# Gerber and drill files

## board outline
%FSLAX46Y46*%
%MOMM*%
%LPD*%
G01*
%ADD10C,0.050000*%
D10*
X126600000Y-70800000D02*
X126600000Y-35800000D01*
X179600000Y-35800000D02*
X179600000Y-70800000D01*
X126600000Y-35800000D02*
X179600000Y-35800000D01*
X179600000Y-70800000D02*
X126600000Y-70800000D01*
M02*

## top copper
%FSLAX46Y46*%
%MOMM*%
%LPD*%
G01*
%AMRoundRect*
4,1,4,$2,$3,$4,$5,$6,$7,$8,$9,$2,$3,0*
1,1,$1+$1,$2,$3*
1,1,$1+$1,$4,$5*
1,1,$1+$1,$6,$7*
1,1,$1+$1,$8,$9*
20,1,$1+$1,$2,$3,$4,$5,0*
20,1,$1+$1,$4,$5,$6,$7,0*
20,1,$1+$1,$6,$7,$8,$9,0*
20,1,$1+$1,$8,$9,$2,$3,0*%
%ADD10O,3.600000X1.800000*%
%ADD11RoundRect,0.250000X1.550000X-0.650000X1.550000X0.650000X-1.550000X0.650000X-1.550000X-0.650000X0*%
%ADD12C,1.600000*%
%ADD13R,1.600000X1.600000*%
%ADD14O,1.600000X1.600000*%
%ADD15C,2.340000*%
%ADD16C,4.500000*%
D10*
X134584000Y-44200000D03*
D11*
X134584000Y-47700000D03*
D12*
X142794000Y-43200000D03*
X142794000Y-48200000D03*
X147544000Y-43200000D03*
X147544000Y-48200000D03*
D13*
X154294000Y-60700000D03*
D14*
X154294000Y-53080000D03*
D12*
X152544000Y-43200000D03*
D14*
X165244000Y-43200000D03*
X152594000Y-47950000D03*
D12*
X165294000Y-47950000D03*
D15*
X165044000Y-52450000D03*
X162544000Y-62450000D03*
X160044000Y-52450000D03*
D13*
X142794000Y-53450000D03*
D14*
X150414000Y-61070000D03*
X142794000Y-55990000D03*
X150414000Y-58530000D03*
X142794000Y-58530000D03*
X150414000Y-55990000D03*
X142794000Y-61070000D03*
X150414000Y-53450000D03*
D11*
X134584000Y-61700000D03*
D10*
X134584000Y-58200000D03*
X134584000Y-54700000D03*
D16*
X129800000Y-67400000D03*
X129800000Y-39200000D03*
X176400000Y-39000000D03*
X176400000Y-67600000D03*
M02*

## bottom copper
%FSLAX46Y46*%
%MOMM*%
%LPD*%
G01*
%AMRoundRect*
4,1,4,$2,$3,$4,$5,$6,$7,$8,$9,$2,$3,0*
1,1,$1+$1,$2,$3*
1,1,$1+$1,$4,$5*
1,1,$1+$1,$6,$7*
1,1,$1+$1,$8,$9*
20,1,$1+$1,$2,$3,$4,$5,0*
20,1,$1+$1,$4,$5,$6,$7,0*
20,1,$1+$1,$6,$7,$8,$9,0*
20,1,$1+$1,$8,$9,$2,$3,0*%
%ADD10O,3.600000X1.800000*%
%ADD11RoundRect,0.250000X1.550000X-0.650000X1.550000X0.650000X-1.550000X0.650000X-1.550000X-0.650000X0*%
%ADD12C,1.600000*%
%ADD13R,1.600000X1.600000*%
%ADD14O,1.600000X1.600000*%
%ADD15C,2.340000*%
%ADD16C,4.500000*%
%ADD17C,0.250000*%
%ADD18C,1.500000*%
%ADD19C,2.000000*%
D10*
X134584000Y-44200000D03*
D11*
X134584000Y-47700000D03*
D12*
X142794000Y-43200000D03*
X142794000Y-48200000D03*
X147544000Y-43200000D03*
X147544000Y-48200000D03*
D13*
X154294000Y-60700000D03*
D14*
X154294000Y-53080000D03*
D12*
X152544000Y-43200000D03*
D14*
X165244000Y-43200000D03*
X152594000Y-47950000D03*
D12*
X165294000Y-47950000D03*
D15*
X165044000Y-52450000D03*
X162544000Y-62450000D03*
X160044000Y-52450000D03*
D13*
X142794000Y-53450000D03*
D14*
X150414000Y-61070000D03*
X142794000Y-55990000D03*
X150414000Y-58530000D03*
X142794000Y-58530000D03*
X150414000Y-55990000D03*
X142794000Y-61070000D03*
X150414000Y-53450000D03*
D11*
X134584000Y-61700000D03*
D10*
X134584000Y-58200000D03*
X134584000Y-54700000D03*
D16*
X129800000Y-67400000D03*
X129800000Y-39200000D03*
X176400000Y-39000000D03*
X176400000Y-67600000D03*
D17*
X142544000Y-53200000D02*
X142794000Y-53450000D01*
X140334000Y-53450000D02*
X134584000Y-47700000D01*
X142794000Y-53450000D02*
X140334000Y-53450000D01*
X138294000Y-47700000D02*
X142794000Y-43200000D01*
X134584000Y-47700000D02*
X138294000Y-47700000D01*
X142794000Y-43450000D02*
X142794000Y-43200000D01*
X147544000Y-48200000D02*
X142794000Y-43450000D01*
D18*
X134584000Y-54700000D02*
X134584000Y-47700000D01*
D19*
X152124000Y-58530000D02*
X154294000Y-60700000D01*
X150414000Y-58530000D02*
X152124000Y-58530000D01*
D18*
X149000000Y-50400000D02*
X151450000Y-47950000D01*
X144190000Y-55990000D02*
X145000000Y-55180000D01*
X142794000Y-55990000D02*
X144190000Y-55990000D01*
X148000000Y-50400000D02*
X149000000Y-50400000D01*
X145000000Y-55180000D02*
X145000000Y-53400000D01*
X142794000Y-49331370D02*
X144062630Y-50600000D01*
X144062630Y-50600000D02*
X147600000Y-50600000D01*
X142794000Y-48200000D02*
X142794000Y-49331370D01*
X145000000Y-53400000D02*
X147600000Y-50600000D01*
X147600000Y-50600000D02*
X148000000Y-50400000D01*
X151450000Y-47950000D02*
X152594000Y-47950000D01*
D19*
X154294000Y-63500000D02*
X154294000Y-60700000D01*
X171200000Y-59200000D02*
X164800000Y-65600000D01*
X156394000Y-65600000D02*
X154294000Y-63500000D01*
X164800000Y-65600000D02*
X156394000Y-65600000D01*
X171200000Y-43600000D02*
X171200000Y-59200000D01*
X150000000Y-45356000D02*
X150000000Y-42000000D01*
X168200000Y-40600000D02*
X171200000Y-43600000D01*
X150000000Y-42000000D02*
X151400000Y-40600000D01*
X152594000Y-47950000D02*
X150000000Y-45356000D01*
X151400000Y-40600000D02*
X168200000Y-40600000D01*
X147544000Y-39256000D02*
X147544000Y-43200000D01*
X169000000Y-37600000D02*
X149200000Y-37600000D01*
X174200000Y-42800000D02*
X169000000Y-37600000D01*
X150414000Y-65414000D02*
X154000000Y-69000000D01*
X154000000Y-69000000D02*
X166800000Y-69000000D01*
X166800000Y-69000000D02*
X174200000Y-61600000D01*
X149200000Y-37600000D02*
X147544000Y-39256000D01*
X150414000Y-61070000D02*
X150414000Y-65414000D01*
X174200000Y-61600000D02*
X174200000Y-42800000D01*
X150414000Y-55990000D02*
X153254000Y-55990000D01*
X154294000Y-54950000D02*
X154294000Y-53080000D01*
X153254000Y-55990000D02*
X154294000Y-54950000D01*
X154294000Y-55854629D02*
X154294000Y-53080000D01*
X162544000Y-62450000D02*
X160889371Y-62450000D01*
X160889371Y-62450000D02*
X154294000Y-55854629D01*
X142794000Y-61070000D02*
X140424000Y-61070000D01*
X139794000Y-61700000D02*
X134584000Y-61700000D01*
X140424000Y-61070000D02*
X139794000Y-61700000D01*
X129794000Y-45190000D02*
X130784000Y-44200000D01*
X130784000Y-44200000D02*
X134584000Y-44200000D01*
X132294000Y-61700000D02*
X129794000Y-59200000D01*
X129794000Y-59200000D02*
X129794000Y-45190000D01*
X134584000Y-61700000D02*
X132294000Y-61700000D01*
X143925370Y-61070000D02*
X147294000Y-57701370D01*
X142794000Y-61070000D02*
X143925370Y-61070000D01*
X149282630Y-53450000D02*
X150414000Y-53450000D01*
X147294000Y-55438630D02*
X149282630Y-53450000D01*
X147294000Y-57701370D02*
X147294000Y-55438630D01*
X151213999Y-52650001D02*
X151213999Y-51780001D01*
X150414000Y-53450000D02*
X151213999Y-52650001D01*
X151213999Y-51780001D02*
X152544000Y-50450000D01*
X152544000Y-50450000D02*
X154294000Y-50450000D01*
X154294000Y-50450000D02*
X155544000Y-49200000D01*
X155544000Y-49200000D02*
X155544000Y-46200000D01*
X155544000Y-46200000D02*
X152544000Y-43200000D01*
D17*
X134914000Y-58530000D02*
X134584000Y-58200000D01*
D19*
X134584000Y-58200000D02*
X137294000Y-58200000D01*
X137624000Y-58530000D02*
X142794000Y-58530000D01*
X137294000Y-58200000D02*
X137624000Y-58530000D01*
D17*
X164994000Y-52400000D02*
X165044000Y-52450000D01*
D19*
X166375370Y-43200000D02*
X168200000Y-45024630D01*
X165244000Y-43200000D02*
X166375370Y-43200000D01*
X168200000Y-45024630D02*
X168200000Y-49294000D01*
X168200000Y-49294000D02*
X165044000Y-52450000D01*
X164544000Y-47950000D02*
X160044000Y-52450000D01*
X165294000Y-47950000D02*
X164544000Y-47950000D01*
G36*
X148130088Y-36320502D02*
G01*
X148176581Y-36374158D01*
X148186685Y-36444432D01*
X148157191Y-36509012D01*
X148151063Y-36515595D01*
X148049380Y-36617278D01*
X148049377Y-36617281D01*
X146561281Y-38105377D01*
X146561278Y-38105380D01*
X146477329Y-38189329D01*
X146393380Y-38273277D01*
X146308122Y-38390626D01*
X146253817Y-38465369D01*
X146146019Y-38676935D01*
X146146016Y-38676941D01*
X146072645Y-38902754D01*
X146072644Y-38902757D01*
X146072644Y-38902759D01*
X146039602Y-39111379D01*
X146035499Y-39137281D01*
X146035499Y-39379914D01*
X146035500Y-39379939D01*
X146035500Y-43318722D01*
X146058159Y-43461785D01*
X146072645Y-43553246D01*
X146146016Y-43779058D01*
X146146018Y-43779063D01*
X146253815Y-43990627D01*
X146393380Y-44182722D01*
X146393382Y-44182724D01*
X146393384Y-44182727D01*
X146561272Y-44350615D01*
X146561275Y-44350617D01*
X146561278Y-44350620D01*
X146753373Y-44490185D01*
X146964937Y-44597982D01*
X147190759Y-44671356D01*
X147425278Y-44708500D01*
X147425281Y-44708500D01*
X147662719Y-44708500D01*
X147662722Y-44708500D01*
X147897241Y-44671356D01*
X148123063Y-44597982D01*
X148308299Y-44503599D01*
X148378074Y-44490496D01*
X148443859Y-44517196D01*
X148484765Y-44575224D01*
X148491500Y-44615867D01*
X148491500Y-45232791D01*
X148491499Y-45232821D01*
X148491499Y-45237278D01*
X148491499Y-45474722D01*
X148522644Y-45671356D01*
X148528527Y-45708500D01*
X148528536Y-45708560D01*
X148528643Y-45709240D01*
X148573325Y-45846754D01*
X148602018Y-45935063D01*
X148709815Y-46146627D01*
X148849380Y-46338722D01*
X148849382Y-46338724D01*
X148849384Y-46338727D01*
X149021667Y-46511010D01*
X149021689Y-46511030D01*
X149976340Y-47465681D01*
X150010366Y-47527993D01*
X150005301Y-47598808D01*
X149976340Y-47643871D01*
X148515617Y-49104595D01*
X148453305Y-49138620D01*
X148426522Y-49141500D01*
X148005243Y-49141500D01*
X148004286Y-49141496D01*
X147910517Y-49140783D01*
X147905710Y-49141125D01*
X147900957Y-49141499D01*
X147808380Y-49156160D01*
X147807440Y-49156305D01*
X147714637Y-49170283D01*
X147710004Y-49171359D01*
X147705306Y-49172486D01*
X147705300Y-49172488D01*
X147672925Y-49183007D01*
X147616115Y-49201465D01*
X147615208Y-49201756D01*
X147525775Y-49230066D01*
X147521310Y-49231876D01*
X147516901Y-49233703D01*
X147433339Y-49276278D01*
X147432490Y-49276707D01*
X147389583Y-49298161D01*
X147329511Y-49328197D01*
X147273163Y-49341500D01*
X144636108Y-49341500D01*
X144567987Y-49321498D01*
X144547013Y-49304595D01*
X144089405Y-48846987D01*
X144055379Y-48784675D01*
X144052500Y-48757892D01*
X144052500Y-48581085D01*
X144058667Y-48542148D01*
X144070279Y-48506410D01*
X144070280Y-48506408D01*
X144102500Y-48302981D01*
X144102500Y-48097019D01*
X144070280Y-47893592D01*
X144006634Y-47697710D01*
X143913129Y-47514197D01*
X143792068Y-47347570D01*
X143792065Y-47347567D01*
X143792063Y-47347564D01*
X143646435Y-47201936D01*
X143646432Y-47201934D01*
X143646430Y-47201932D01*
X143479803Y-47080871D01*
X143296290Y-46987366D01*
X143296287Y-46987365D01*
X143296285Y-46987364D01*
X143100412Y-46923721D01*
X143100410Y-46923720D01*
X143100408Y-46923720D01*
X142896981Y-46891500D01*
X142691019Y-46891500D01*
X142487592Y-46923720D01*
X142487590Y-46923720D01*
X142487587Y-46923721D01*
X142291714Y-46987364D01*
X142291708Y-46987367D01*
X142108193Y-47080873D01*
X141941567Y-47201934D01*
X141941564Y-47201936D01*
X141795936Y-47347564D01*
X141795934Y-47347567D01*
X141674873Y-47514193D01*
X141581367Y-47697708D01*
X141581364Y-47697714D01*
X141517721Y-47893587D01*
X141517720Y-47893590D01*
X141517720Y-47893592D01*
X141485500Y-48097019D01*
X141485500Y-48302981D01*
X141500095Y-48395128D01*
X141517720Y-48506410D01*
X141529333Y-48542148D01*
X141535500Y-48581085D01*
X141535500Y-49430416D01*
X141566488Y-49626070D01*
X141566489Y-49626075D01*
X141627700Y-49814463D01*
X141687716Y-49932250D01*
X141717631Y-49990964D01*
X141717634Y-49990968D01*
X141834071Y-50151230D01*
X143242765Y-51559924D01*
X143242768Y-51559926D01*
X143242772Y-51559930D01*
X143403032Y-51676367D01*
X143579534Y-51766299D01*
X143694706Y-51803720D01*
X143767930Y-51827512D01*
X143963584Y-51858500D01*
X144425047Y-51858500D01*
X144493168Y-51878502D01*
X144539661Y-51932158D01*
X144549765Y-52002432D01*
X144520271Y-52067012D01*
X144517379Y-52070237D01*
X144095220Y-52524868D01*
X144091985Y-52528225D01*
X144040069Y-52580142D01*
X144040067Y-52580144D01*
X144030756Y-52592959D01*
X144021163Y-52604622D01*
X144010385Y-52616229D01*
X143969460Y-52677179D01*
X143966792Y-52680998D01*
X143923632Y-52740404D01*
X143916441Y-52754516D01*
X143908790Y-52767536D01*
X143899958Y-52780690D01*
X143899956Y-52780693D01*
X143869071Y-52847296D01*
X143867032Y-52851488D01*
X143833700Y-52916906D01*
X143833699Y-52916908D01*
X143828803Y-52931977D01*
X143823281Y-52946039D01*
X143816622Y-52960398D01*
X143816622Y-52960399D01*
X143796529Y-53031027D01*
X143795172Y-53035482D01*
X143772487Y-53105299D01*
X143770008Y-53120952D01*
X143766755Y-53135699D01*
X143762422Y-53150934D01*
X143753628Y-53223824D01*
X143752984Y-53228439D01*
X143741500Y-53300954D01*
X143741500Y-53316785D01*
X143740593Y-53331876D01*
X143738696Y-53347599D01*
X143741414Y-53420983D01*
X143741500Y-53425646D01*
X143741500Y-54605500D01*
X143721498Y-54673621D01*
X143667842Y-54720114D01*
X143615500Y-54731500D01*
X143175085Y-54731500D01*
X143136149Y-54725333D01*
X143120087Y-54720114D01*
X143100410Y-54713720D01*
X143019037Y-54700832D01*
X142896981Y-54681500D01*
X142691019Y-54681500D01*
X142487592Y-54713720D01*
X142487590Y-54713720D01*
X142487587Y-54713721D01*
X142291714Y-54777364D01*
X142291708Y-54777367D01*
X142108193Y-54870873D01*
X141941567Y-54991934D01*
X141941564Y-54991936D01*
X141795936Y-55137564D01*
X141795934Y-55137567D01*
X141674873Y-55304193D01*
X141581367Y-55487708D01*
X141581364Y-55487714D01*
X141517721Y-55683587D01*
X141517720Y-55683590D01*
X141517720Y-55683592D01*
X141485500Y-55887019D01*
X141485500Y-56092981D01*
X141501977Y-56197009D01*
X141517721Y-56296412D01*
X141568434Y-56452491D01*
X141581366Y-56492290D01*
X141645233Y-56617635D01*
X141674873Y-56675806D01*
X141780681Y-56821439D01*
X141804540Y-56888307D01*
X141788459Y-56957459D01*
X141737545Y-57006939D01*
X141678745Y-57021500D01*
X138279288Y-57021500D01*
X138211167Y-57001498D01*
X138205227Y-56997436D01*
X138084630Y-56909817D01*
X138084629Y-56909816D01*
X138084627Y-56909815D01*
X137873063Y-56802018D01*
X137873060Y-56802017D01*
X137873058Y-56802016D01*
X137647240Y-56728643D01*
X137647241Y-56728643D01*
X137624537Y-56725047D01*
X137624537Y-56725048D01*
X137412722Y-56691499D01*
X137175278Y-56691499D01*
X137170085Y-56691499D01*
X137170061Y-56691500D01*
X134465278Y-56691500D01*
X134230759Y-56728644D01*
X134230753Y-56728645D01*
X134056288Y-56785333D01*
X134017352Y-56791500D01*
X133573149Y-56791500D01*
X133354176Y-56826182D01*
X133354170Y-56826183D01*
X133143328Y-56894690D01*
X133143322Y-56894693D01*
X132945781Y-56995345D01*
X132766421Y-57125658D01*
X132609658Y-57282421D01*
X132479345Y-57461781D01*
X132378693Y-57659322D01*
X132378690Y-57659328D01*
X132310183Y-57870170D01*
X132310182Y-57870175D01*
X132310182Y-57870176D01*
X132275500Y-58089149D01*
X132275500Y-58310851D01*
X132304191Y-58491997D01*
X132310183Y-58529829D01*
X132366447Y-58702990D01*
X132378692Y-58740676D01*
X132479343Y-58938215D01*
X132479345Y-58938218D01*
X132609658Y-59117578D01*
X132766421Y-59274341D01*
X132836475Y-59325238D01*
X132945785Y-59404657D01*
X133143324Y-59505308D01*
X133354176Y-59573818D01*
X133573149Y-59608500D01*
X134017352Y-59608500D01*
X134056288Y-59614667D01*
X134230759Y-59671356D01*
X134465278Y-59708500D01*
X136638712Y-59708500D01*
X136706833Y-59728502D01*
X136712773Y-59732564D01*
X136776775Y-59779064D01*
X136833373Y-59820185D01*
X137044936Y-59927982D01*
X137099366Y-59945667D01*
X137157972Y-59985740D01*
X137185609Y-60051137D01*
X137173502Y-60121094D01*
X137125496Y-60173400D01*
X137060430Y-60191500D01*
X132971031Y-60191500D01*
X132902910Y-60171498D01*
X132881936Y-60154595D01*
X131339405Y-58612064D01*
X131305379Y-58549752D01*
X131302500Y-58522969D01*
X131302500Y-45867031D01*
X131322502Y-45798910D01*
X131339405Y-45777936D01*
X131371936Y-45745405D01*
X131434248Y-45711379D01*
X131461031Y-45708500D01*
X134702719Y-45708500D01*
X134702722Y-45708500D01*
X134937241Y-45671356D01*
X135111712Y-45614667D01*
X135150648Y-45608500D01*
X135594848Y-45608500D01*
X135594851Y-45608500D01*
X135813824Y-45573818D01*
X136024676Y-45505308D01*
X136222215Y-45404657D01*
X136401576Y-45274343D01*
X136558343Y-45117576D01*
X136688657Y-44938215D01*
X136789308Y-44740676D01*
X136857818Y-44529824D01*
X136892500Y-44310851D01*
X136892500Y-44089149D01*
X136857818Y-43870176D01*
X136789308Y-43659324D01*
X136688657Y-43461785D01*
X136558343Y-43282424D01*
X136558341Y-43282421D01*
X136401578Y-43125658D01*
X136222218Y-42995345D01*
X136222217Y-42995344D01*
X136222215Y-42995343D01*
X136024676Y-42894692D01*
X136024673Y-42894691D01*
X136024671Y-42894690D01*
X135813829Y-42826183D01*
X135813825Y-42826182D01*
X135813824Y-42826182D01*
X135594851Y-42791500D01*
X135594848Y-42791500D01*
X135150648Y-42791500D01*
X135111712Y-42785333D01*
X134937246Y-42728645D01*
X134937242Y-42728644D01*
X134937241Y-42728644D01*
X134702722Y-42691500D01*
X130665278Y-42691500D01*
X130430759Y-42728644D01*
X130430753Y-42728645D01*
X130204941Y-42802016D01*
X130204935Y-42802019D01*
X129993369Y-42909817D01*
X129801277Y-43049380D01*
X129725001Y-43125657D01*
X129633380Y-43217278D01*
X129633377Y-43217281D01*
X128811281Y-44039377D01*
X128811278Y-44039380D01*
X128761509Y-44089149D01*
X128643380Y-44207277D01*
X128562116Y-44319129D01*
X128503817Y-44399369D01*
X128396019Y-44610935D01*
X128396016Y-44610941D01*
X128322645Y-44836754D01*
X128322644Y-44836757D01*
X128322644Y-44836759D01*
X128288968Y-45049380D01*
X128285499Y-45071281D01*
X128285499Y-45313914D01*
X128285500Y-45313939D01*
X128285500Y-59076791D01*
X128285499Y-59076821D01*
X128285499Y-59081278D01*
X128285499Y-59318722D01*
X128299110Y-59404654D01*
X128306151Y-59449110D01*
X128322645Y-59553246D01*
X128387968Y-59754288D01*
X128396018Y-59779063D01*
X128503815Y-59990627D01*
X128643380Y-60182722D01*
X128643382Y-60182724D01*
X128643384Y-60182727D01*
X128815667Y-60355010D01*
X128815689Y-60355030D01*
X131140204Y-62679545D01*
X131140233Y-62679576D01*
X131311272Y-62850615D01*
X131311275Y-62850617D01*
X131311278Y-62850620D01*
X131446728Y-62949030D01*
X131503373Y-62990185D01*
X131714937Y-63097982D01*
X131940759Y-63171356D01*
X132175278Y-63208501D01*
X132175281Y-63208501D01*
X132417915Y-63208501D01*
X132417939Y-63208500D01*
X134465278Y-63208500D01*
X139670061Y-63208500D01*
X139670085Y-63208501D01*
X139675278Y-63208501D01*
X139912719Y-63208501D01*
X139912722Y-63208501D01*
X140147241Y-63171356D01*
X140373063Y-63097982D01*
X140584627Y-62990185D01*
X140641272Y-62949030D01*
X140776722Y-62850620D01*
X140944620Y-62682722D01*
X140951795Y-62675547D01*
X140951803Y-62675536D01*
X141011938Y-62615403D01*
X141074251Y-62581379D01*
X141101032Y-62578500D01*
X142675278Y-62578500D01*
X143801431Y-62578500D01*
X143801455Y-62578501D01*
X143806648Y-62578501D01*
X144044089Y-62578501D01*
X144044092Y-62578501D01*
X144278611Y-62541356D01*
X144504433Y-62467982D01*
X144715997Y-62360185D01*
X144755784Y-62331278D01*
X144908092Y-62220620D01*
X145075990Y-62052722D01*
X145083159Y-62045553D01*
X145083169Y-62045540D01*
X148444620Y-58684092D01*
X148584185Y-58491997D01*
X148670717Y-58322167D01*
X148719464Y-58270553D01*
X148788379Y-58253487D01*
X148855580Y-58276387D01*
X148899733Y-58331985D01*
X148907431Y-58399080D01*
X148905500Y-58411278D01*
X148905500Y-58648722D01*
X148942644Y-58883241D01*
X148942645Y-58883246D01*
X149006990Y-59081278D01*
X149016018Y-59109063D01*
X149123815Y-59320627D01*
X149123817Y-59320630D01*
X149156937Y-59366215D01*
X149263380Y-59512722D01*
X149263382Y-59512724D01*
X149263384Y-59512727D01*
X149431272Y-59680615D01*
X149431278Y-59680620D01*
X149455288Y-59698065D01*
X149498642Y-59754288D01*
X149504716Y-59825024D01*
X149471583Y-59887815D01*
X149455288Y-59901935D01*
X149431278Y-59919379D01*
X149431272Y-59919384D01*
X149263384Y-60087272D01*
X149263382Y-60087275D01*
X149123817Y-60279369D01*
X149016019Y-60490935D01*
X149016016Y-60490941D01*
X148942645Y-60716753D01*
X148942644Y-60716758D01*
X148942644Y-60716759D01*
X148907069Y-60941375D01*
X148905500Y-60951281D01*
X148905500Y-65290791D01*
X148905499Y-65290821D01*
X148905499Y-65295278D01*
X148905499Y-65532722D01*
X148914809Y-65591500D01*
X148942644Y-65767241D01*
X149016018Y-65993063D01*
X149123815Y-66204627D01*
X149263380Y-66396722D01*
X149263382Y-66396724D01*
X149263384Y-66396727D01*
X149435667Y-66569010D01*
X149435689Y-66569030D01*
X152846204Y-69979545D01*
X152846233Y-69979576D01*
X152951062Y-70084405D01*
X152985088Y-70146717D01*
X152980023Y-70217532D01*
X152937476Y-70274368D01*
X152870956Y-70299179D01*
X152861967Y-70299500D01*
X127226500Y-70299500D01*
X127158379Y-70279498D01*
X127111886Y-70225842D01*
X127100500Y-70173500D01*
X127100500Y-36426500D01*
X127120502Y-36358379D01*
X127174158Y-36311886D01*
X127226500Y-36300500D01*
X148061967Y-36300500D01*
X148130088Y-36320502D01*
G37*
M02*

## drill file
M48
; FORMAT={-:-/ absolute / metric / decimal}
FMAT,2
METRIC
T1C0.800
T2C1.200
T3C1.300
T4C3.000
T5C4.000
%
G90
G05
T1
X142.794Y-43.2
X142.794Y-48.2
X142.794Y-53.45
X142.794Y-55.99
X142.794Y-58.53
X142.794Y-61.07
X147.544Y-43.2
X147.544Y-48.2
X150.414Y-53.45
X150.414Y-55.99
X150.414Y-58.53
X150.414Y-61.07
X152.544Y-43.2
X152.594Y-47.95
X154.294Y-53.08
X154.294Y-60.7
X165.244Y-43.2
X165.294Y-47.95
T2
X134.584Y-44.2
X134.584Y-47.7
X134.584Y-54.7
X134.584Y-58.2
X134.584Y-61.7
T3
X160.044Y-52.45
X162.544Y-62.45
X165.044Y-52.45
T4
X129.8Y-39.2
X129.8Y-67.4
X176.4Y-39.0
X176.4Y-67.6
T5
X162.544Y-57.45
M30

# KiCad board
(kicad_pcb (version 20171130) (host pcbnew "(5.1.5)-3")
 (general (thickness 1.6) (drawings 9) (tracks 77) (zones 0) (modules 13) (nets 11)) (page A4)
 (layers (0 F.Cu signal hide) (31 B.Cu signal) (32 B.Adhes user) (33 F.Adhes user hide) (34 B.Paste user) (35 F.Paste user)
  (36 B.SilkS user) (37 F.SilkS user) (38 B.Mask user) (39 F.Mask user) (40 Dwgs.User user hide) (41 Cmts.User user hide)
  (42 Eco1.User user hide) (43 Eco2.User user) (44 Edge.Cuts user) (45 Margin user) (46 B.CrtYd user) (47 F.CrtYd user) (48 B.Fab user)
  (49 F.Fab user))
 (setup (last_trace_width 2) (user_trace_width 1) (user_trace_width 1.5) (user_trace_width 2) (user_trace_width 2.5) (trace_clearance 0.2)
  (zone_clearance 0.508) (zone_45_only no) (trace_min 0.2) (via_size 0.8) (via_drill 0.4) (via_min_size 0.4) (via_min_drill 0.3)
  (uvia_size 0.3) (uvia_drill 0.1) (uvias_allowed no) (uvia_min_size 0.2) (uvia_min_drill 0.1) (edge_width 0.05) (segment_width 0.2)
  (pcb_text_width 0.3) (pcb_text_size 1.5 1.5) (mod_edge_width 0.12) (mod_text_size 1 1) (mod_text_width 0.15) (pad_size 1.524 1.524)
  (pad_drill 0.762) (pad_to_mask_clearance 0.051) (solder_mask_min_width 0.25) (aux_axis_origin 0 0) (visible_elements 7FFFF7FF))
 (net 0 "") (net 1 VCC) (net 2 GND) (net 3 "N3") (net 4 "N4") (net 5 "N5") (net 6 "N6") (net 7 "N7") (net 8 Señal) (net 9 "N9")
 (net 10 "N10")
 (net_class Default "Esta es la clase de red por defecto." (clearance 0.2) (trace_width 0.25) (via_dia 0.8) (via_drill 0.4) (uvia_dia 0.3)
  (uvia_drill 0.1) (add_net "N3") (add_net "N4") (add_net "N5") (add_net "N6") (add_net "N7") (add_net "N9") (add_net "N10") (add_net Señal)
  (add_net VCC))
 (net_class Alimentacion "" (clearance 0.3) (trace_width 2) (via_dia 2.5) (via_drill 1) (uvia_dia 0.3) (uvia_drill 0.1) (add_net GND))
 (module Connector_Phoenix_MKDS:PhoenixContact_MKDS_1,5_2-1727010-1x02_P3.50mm (layer F.Cu) (at 132.044 47.7 90)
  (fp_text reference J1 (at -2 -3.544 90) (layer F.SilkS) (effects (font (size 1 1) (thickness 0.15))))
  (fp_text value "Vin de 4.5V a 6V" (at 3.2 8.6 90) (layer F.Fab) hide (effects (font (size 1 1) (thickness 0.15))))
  (pad 2 thru_hole oval (at 3.5 2.54 90) (size 1.8 3.6) (drill 1.2) (layers *.Cu *.Mask) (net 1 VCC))
  (pad 1 thru_hole roundrect (at 0 2.54 90) (size 1.8 3.6) (drill 1.2) (layers *.Cu *.Mask) (roundrect_rratio 0.138889) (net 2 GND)))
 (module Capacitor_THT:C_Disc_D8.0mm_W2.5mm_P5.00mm (layer F.Cu) (at 142.794 48.2 90)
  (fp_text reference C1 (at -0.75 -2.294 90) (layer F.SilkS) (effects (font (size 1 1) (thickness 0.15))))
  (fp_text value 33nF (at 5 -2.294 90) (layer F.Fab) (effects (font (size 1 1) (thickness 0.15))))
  (pad 2 thru_hole circle (at 5 0 90) (size 1.6 1.6) (drill 0.8) (layers *.Cu *.Mask) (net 2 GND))
  (pad 1 thru_hole circle (at 0 0 90) (size 1.6 1.6) (drill 0.8) (layers *.Cu *.Mask) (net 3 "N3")))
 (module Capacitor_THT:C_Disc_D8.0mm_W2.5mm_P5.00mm (layer F.Cu) (at 147.544 43.2 270)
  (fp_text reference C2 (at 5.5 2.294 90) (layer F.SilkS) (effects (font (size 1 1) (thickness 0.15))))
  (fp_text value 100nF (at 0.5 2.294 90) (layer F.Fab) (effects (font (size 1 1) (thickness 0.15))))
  (pad 1 thru_hole circle (at 0 0 270) (size 1.6 1.6) (drill 0.8) (layers *.Cu *.Mask) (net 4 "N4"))
  (pad 2 thru_hole circle (at 5 0 270) (size 1.6 1.6) (drill 0.8) (layers *.Cu *.Mask) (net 2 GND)))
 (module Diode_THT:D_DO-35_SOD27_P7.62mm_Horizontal (layer F.Cu) (at 154.294 60.7 90)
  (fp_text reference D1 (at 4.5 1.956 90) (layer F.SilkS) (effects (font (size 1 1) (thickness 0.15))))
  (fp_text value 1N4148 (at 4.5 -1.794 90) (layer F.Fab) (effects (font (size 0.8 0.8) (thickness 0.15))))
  (pad 1 thru_hole rect (at 0 0 90) (size 1.6 1.6) (drill 0.8) (layers *.Cu *.Mask) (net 3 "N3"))
  (pad 2 thru_hole oval (at 7.62 0 90) (size 1.6 1.6) (drill 0.8) (layers *.Cu *.Mask) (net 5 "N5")))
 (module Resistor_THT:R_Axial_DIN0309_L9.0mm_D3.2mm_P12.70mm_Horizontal (layer F.Cu) (at 152.544 43.2)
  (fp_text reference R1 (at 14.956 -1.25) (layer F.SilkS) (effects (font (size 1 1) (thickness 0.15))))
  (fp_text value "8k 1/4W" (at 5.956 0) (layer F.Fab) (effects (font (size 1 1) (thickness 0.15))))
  (pad 1 thru_hole circle (at 0 0) (size 1.6 1.6) (drill 0.8) (layers *.Cu *.Mask) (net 1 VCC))
  (pad 2 thru_hole oval (at 12.7 0) (size 1.6 1.6) (drill 0.8) (layers *.Cu *.Mask) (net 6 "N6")))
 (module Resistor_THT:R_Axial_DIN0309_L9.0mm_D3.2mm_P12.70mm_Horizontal (layer F.Cu) (at 165.294 47.95 180)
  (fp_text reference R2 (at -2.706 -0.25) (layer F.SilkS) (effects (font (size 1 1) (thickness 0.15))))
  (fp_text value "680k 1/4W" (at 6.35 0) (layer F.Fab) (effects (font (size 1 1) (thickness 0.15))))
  (pad 2 thru_hole oval (at 12.7 0 180) (size 1.6 1.6) (drill 0.8) (layers *.Cu *.Mask) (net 3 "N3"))
  (pad 1 thru_hole circle (at 0 0 180) (size 1.6 1.6) (drill 0.8) (layers *.Cu *.Mask) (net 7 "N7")))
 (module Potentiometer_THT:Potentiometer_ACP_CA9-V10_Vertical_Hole (layer F.Cu) (at 160.044 52.45 270)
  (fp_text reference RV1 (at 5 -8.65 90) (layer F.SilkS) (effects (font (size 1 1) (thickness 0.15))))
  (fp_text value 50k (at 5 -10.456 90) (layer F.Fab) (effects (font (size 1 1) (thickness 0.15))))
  (pad 3 thru_hole circle (at 0 -5 270) (size 2.34 2.34) (drill 1.3) (layers *.Cu *.Mask) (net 6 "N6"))
  (pad 2 thru_hole circle (at 10 -2.5 270) (size 2.34 2.34) (drill 1.3) (layers *.Cu *.Mask) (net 5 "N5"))
  (pad 1 thru_hole circle (at 0 0 270) (size 2.34 2.34) (drill 1.3) (layers *.Cu *.Mask) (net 7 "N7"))
  (pad "" np_thru_hole circle (at 5 -2.5 270) (size 4 4) (drill 4) (layers *.Cu *.Mask)))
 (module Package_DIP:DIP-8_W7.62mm (layer F.Cu) (at 142.794 53.45)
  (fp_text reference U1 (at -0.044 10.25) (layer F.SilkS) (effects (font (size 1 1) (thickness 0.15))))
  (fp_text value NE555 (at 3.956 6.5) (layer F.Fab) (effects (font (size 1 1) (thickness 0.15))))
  (pad 1 thru_hole rect (at 0 0) (size 1.6 1.6) (drill 0.8) (layers *.Cu *.Mask) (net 2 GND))
  (pad 5 thru_hole oval (at 7.62 7.62) (size 1.6 1.6) (drill 0.8) (layers *.Cu *.Mask) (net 4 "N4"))
  (pad 2 thru_hole oval (at 0 2.54) (size 1.6 1.6) (drill 0.8) (layers *.Cu *.Mask) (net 3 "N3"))
  (pad 6 thru_hole oval (at 7.62 5.08) (size 1.6 1.6) (drill 0.8) (layers *.Cu *.Mask) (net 3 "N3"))
  (pad 3 thru_hole oval (at 0 5.08) (size 1.6 1.6) (drill 0.8) (layers *.Cu *.Mask) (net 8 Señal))
  (pad 7 thru_hole oval (at 7.62 2.54) (size 1.6 1.6) (drill 0.8) (layers *.Cu *.Mask) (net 5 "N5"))
  (pad 4 thru_hole oval (at 0 7.62) (size 1.6 1.6) (drill 0.8) (layers *.Cu *.Mask) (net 1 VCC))
  (pad 8 thru_hole oval (at 7.62 0) (size 1.6 1.6) (drill 0.8) (layers *.Cu *.Mask) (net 1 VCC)))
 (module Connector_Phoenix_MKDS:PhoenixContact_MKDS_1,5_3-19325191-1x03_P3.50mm (layer F.Cu) (at 132.044 61.7 90)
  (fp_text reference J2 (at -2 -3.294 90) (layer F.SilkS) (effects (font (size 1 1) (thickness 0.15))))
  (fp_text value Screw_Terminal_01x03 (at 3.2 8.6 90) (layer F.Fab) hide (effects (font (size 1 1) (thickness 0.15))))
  (pad 1 thru_hole roundrect (at 0 2.54 90) (size 1.8 3.6) (drill 1.2) (layers *.Cu *.Mask) (roundrect_rratio 0.138889) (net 1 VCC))
  (pad 2 thru_hole oval (at 3.5 2.54 90) (size 1.8 3.6) (drill 1.2) (layers *.Cu *.Mask) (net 8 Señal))
  (pad 3 thru_hole oval (at 7 2.54 90) (size 1.8 3.6) (drill 1.2) (layers *.Cu *.Mask) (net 2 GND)))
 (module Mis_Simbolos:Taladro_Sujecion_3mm (layer F.Cu) (at 129.8 67.4)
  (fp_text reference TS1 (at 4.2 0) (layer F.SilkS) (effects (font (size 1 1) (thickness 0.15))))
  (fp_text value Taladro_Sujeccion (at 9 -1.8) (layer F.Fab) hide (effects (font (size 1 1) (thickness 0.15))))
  (pad 1 thru_hole circle (at 0 0) (size 4.5 4.5) (drill 3) (layers *.Cu *.Mask) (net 2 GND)))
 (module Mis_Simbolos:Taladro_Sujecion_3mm (layer F.Cu) (at 129.8 39.2)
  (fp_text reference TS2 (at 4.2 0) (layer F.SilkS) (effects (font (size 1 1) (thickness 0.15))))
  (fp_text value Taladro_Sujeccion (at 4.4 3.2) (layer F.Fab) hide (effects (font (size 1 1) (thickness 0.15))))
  (pad 1 thru_hole circle (at 0 0) (size 4.5 4.5) (drill 3) (layers *.Cu *.Mask) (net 2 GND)))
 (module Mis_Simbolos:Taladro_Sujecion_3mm (layer F.Cu) (at 176.4 39)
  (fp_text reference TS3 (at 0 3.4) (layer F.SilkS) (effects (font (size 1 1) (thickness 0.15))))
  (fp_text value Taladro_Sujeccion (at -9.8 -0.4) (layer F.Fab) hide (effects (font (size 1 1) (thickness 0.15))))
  (pad 1 thru_hole circle (at 0 0) (size 4.5 4.5) (drill 3) (layers *.Cu *.Mask) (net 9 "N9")))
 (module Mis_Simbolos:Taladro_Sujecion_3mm (layer F.Cu) (at 176.4 67.6)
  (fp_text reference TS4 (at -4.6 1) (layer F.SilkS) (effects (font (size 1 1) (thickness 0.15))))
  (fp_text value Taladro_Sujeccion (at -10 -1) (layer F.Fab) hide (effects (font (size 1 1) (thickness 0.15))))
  (pad 1 thru_hole circle (at 0 0) (size 4.5 4.5) (drill 3) (layers *.Cu *.Mask) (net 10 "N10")))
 (gr_line (start 126.6 70.8) (end 126.6 35.8) (layer Edge.Cuts) (width 0.05))
 (gr_line (start 179.6 35.8) (end 179.6 70.8) (layer Edge.Cuts) (width 0.05))
 (gr_line (start 126.6 35.8) (end 179.6 35.8) (layer Edge.Cuts) (width 0.05))
 (gr_line (start 179.6 70.8) (end 126.6 70.8) (layer Edge.Cuts) (width 0.05))
 (segment (start 142.544 53.2) (end 142.794 53.45) (width 0.25) (layer B.Cu) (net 2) (status 30))
 (segment (start 140.334 53.45) (end 134.584 47.7) (width 0.25) (layer B.Cu) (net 2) (status 20))
 (segment (start 142.794 53.45) (end 140.334 53.45) (width 0.25) (layer B.Cu) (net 2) (status 10))
 (segment (start 138.294 47.7) (end 142.794 43.2) (width 0.25) (layer B.Cu) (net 2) (status 20))
 (segment (start 134.584 47.7) (end 138.294 47.7) (width 0.25) (layer B.Cu) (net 2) (status 10))
 (segment (start 142.794 43.45) (end 142.794 43.2) (width 0.25) (layer B.Cu) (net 2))
 (segment (start 147.544 48.2) (end 142.794 43.45) (width 0.25) (layer B.Cu) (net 2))
 (segment (start 134.584 54.7) (end 134.584 47.7) (width 1.5) (layer B.Cu) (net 2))
 (segment (start 152.124 58.53) (end 154.294 60.7) (width 2) (layer B.Cu) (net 3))
 (segment (start 150.414 58.53) (end 152.124 58.53) (width 2) (layer B.Cu) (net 3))
 (segment (start 149 50.4) (end 151.45 47.95) (width 1.5) (layer B.Cu) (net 3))
 (segment (start 144.19 55.99) (end 145 55.18) (width 1.5) (layer B.Cu) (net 3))
 (segment (start 142.794 55.99) (end 144.19 55.99) (width 1.5) (layer B.Cu) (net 3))
 (segment (start 148 50.4) (end 149 50.4) (width 1.5) (layer B.Cu) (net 3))
 (segment (start 145 55.18) (end 145 53.4) (width 1.5) (layer B.Cu) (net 3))
 (segment (start 142.794 49.33137) (end 144.06263 50.6) (width 1.5) (layer B.Cu) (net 3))
 (segment (start 144.06263 50.6) (end 147.6 50.6) (width 1.5) (layer B.Cu) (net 3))
 (segment (start 142.794 48.2) (end 142.794 49.33137) (width 1.5) (layer B.Cu) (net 3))
 (segment (start 145 53.4) (end 147.6 50.6) (width 1.5) (layer B.Cu) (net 3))
 (segment (start 147.6 50.6) (end 148 50.4) (width 1.5) (layer B.Cu) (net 3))
 (segment (start 151.45 47.95) (end 152.594 47.95) (width 1.5) (layer B.Cu) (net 3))
 (segment (start 154.294 63.5) (end 154.294 60.7) (width 2) (layer B.Cu) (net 3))
 (segment (start 171.2 59.2) (end 164.8 65.6) (width 2) (layer B.Cu) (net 3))
 (segment (start 156.394 65.6) (end 154.294 63.5) (width 2) (layer B.Cu) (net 3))
 (segment (start 164.8 65.6) (end 156.394 65.6) (width 2) (layer B.Cu) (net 3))
 (segment (start 171.2 43.6) (end 171.2 59.2) (width 2) (layer B.Cu) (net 3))
 (segment (start 150 45.356) (end 150 42) (width 2) (layer B.Cu) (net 3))
 (segment (start 168.2 40.6) (end 171.2 43.6) (width 2) (layer B.Cu) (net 3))
 (segment (start 150 42) (end 151.4 40.6) (width 2) (layer B.Cu) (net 3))
 (segment (start 152.594 47.95) (end 150 45.356) (width 2) (layer B.Cu) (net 3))
 (segment (start 151.4 40.6) (end 168.2 40.6) (width 2) (layer B.Cu) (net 3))
 (segment (start 147.544 39.256) (end 147.544 43.2) (width 2) (layer B.Cu) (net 4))
 (segment (start 169 37.6) (end 149.2 37.6) (width 2) (layer B.Cu) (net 4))
 (segment (start 174.2 42.8) (end 169 37.6) (width 2) (layer B.Cu) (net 4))
 (segment (start 150.414 65.414) (end 154 69) (width 2) (layer B.Cu) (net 4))
 (segment (start 154 69) (end 166.8 69) (width 2) (layer B.Cu) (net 4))
 (segment (start 166.8 69) (end 174.2 61.6) (width 2) (layer B.Cu) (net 4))
 (segment (start 149.2 37.6) (end 147.544 39.256) (width 2) (layer B.Cu) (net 4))
 (segment (start 150.414 61.07) (end 150.414 65.414) (width 2) (layer B.Cu) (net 4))
 (segment (start 174.2 61.6) (end 174.2 42.8) (width 2) (layer B.Cu) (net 4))
 (segment (start 150.414 55.99) (end 153.254 55.99) (width 2) (layer B.Cu) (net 5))
 (segment (start 154.294 54.95) (end 154.294 53.08) (width 2) (layer B.Cu) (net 5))
 (segment (start 153.254 55.99) (end 154.294 54.95) (width 2) (layer B.Cu) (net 5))
 (segment (start 154.294 55.854629) (end 154.294 53.08) (width 2) (layer B.Cu) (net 5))
 (segment (start 162.544 62.45) (end 160.889371 62.45) (width 2) (layer B.Cu) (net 5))
 (segment (start 160.889371 62.45) (end 154.294 55.854629) (width 2) (layer B.Cu) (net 5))
 (segment (start 142.794 61.07) (end 140.424 61.07) (width 2) (layer B.Cu) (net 1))
 (segment (start 139.794 61.7) (end 134.584 61.7) (width 2) (layer B.Cu) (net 1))
 (segment (start 140.424 61.07) (end 139.794 61.7) (width 2) (layer B.Cu) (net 1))
 (segment (start 129.794 45.19) (end 130.784 44.2) (width 2) (layer B.Cu) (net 1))
 (segment (start 130.784 44.2) (end 134.584 44.2) (width 2) (layer B.Cu) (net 1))
 (segment (start 132.294 61.7) (end 129.794 59.2) (width 2) (layer B.Cu) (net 1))
 (segment (start 129.794 59.2) (end 129.794 45.19) (width 2) (layer B.Cu) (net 1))
 (segment (start 134.584 61.7) (end 132.294 61.7) (width 2) (layer B.Cu) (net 1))
 (segment (start 143.92537 61.07) (end 147.294 57.70137) (width 2) (layer B.Cu) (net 1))
 (segment (start 142.794 61.07) (end 143.92537 61.07) (width 2) (layer B.Cu) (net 1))
 (segment (start 149.28263 53.45) (end 150.414 53.45) (width 2) (layer B.Cu) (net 1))
 (segment (start 147.294 55.43863) (end 149.28263 53.45) (width 2) (layer B.Cu) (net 1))
 (segment (start 147.294 57.70137) (end 147.294 55.43863) (width 2) (layer B.Cu) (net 1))
 (segment (start 151.213999 52.650001) (end 151.213999 51.780001) (width 2) (layer B.Cu) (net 1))
 (segment (start 150.414 53.45) (end 151.213999 52.650001) (width 2) (layer B.Cu) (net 1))
 (segment (start 151.213999 51.780001) (end 152.544 50.45) (width 2) (layer B.Cu) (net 1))
 (segment (start 152.544 50.45) (end 154.294 50.45) (width 2) (layer B.Cu) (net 1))
 (segment (start 154.294 50.45) (end 155.544 49.2) (width 2) (layer B.Cu) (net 1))
 (segment (start 155.544 49.2) (end 155.544 46.2) (width 2) (layer B.Cu) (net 1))
 (segment (start 155.544 46.2) (end 152.544 43.2) (width 2) (layer B.Cu) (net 1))
 (segment (start 134.914 58.53) (end 134.584 58.2) (width 0.25) (layer B.Cu) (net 8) (status 30))
 (segment (start 134.584 58.2) (end 137.294 58.2) (width 2) (layer B.Cu) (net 8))
 (segment (start 137.624 58.53) (end 142.794 58.53) (width 2) (layer B.Cu) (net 8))
 (segment (start 137.294 58.2) (end 137.624 58.53) (width 2) (layer B.Cu) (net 8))
 (segment (start 164.994 52.4) (end 165.044 52.45) (width 0.25) (layer B.Cu) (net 6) (status 30))
 (segment (start 166.37537 43.2) (end 168.2 45.02463) (width 2) (layer B.Cu) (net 6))
 (segment (start 165.244 43.2) (end 166.37537 43.2) (width 2) (layer B.Cu) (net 6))
 (segment (start 168.2 45.02463) (end 168.2 49.294) (width 2) (layer B.Cu) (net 6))
 (segment (start 168.2 49.294) (end 165.044 52.45) (width 2) (layer B.Cu) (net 6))
 (segment (start 164.544 47.95) (end 160.044 52.45) (width 2) (layer B.Cu) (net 7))
 (segment (start 165.294 47.95) (end 164.544 47.95) (width 2) (layer B.Cu) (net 7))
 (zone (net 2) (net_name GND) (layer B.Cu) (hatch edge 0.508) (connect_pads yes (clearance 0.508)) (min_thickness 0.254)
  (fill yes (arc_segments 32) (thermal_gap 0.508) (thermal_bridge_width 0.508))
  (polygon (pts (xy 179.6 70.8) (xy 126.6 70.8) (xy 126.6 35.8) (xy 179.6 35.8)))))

